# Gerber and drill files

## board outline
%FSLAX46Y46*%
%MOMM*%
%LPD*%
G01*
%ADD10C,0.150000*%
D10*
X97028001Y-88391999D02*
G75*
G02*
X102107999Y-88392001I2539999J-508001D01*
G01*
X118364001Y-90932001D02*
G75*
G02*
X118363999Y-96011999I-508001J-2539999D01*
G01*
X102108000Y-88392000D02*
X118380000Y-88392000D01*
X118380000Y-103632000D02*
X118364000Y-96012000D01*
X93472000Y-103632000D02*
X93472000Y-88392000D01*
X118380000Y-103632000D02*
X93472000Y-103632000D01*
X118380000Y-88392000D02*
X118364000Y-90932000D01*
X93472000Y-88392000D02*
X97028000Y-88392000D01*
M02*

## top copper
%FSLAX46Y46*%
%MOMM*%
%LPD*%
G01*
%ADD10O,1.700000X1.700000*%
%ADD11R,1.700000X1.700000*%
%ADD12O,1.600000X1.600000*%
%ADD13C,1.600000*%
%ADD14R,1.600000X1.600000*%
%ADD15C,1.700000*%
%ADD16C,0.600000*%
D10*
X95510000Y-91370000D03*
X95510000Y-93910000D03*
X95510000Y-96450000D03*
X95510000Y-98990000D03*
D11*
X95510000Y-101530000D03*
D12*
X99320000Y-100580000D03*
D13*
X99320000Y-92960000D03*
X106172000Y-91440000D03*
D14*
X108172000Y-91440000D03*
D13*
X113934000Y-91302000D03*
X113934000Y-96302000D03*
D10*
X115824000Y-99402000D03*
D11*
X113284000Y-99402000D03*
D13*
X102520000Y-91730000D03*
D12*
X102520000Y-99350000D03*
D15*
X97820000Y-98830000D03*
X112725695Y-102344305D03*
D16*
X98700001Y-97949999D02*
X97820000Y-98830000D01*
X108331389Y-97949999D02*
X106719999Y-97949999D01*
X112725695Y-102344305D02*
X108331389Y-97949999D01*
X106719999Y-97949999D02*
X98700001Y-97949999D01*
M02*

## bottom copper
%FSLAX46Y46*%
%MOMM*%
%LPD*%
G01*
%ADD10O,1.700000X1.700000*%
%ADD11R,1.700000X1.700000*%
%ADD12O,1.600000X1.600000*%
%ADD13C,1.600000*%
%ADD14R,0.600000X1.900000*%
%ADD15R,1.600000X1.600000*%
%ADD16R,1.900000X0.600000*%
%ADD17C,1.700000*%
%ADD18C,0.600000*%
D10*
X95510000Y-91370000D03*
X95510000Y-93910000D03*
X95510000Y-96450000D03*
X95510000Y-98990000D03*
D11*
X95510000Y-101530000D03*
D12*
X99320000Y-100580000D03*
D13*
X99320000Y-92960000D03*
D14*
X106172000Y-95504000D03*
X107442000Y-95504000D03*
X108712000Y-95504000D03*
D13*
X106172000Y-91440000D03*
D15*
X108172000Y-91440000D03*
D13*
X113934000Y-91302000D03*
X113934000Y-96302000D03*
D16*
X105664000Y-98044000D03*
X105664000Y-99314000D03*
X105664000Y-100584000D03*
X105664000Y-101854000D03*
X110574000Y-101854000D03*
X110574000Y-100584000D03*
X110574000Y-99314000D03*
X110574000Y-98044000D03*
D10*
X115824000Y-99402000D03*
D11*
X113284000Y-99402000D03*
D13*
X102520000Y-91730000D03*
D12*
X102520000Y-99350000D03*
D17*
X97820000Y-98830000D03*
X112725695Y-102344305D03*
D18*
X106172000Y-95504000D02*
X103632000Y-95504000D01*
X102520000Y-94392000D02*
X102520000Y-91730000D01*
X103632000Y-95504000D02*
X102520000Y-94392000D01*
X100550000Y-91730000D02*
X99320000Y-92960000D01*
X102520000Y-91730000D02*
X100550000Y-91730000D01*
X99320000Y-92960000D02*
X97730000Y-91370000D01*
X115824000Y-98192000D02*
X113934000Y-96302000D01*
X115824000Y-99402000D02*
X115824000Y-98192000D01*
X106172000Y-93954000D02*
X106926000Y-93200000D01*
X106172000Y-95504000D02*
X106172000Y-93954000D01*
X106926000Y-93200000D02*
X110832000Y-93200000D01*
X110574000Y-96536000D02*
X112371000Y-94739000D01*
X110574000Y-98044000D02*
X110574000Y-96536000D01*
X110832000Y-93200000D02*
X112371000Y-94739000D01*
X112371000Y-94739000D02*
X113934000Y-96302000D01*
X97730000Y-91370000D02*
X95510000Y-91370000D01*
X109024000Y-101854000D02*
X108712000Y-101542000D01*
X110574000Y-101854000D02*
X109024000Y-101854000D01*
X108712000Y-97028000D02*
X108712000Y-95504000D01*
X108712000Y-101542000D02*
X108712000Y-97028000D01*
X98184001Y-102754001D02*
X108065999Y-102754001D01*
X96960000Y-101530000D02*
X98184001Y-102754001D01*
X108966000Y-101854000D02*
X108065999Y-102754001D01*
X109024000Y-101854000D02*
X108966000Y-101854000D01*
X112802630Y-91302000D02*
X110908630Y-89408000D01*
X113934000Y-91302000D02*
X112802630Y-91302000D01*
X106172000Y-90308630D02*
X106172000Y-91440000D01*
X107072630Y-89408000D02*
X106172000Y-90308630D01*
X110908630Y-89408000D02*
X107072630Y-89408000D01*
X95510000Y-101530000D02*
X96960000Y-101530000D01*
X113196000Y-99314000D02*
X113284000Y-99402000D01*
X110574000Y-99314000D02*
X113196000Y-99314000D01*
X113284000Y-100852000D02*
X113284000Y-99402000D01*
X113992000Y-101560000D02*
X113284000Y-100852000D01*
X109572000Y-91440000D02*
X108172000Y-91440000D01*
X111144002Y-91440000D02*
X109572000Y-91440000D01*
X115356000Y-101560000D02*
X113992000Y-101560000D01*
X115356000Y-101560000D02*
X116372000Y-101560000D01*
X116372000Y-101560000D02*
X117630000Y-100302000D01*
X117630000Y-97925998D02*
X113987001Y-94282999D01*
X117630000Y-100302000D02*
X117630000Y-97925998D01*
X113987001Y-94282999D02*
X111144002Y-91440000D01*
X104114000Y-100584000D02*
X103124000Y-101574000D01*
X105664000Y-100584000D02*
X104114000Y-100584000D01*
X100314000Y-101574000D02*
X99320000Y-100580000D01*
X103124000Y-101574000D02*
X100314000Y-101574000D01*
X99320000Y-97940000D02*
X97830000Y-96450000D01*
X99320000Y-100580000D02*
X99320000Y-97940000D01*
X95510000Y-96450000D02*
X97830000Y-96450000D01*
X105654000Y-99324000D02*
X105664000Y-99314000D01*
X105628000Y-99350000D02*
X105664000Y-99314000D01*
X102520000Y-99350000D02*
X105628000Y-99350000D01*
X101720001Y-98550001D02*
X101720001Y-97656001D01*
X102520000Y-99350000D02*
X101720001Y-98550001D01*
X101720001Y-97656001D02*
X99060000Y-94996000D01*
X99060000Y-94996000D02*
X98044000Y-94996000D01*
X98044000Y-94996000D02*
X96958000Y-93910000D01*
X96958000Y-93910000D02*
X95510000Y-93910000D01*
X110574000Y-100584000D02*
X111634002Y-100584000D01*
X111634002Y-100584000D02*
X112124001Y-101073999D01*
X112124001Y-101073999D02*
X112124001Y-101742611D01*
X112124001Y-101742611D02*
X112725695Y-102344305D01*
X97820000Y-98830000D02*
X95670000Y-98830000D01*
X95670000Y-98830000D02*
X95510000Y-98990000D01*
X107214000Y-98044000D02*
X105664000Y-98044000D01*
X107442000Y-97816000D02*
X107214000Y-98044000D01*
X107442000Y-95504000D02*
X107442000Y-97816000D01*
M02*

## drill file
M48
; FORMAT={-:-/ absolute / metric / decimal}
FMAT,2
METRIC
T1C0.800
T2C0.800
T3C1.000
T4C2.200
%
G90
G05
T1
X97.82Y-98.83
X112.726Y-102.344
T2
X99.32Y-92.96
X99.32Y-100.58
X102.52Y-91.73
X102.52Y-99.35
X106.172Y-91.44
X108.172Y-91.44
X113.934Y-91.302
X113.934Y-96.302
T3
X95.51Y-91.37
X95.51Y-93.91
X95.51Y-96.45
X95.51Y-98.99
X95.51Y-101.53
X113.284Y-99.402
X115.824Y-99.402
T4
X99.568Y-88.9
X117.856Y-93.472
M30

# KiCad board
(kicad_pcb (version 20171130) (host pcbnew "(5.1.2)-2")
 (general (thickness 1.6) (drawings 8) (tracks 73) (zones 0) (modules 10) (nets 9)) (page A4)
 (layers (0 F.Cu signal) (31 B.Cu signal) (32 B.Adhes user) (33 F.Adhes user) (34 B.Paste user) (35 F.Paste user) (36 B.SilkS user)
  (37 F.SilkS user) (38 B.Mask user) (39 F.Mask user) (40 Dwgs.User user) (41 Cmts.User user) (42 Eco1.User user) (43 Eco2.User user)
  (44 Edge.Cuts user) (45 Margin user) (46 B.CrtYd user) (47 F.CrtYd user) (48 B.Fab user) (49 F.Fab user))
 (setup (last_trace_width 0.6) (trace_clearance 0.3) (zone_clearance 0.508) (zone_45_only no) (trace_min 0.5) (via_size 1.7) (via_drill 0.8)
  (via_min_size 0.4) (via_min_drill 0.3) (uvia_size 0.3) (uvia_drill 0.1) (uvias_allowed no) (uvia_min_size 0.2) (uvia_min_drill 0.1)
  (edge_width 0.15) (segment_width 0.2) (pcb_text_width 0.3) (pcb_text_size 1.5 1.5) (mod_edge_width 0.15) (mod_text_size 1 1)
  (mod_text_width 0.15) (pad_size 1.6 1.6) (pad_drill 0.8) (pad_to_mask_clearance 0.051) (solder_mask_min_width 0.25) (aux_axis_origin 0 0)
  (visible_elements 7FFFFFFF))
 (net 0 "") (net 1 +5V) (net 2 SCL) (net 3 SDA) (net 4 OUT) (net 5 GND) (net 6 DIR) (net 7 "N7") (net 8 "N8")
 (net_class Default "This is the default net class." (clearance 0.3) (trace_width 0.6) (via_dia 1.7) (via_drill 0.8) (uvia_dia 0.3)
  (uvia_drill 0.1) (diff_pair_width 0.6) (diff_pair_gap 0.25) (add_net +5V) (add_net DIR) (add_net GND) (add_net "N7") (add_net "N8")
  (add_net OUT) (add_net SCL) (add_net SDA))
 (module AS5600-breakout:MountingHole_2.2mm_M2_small (layer F.Cu) (at 99.568 88.9)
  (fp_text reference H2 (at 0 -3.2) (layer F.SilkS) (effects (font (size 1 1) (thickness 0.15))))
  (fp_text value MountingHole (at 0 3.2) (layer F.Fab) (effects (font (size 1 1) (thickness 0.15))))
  (pad 1 np_thru_hole circle (at 0 0) (size 2.2 2.2) (drill 2.2) (layers *.Cu *.Mask)))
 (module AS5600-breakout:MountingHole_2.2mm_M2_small (layer F.Cu) (at 117.856 93.472)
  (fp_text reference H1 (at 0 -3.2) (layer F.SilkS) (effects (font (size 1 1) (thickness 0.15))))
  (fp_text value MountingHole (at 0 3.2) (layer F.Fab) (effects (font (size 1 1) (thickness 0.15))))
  (pad 1 np_thru_hole circle (at 0 0) (size 2.2 2.2) (drill 2.2) (layers *.Cu *.Mask)))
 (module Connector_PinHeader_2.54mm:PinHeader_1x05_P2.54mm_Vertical (layer F.Cu) (at 95.51 101.53 180)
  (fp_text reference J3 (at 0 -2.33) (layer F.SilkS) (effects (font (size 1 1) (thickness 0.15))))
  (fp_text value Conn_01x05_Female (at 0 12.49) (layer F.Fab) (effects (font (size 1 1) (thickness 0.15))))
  (pad 5 thru_hole oval (at 0 10.16 180) (size 1.7 1.7) (drill 1) (layers *.Cu *.Mask) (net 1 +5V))
  (pad 4 thru_hole oval (at 0 7.62 180) (size 1.7 1.7) (drill 1) (layers *.Cu *.Mask) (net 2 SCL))
  (pad 3 thru_hole oval (at 0 5.08 180) (size 1.7 1.7) (drill 1) (layers *.Cu *.Mask) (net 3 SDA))
  (pad 2 thru_hole oval (at 0 2.54 180) (size 1.7 1.7) (drill 1) (layers *.Cu *.Mask) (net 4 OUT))
  (pad 1 thru_hole rect (at 0 0 180) (size 1.7 1.7) (drill 1) (layers *.Cu *.Mask) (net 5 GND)))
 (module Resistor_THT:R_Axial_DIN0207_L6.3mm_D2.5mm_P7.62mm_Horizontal (layer F.Cu) (at 99.32 92.96 270)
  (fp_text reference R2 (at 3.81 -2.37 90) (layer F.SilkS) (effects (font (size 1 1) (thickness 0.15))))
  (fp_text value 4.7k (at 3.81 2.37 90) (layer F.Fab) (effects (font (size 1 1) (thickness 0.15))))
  (pad 2 thru_hole oval (at 7.62 0 270) (size 1.6 1.6) (drill 0.8) (layers *.Cu *.Mask) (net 3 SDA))
  (pad 1 thru_hole circle (at 0 0 270) (size 1.6 1.6) (drill 0.8) (layers *.Cu *.Mask) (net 1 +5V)))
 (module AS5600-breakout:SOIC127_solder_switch (layer B.Cu) (at 106.807 93.049 90)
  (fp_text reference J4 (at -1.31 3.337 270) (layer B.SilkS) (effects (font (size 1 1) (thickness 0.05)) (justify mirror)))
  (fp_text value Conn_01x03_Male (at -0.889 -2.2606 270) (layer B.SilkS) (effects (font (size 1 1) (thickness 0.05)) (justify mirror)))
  (pad 3 smd rect (at -2.455 -0.635 90) (size 1.9 0.6) (layers B.Cu B.Paste B.Mask) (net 1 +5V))
  (pad 2 smd rect (at -2.455 0.635 90) (size 1.9 0.6) (layers B.Cu B.Paste B.Mask) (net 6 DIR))
  (pad 1 smd rect (at -2.455 1.905 90) (size 1.9 0.6) (layers B.Cu B.Paste B.Mask) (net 5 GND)))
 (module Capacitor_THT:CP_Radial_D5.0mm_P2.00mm (layer F.Cu) (at 108.172 91.44 180)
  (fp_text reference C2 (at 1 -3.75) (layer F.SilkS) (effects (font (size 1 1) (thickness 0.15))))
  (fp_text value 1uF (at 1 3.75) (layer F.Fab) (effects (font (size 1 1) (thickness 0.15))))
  (pad 2 thru_hole circle (at 2 0 180) (size 1.6 1.6) (drill 0.8) (layers *.Cu *.Mask) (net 5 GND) (clearance 0.2))
  (pad 1 thru_hole rect (at 0 0 180) (size 1.6 1.6) (drill 0.8) (layers *.Cu *.Mask) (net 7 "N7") (clearance 0.2)))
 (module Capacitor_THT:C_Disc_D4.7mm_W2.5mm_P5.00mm (layer F.Cu) (at 113.934 96.302 90)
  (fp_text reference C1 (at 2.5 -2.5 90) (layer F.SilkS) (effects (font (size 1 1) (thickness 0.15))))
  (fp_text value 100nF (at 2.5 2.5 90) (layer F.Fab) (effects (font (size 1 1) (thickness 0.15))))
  (pad 2 thru_hole circle (at 5 0 90) (size 1.6 1.6) (drill 0.8) (layers *.Cu *.Mask) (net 5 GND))
  (pad 1 thru_hole circle (at 0 0 90) (size 1.6 1.6) (drill 0.8) (layers *.Cu *.Mask) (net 1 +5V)))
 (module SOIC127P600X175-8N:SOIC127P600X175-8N (layer B.Cu) (at 108.119 99.949 180)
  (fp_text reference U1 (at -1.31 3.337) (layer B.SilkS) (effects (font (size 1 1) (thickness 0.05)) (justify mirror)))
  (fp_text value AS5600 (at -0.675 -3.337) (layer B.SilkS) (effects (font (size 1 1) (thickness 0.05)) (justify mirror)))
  (pad 8 smd rect (at 2.455 1.905 180) (size 1.9 0.6) (layers B.Cu B.Paste B.Mask) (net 6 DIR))
  (pad 7 smd rect (at 2.455 0.635 180) (size 1.9 0.6) (layers B.Cu B.Paste B.Mask) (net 2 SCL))
  (pad 6 smd rect (at 2.455 -0.635 180) (size 1.9 0.6) (layers B.Cu B.Paste B.Mask) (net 3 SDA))
  (pad 5 smd rect (at 2.455 -1.905 180) (size 1.9 0.6) (layers B.Cu B.Paste B.Mask) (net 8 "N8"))
  (pad 4 smd rect (at -2.455 -1.905 180) (size 1.9 0.6) (layers B.Cu B.Paste B.Mask) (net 5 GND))
  (pad 3 smd rect (at -2.455 -0.635 180) (size 1.9 0.6) (layers B.Cu B.Paste B.Mask) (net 4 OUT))
  (pad 2 smd rect (at -2.455 0.635 180) (size 1.9 0.6) (layers B.Cu B.Paste B.Mask) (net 7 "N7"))
  (pad 1 smd rect (at -2.455 1.905 180) (size 1.9 0.6) (layers B.Cu B.Paste B.Mask) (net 1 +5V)))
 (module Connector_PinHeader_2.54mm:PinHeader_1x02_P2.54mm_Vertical (layer F.Cu) (at 113.284 99.402 90)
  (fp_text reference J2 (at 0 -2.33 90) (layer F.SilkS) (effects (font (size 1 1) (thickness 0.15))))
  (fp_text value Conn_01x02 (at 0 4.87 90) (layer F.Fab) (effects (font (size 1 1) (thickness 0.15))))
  (pad 2 thru_hole oval (at 0 2.54 90) (size 1.7 1.7) (drill 1) (layers *.Cu *.Mask) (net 1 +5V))
  (pad 1 thru_hole rect (at 0 0 90) (size 1.7 1.7) (drill 1) (layers *.Cu *.Mask) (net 7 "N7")))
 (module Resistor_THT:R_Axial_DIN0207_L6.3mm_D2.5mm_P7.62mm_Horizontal (layer F.Cu) (at 102.52 91.73 270)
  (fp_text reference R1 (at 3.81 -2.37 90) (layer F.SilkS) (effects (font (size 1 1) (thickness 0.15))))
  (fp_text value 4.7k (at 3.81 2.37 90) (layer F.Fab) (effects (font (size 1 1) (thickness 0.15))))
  (pad 1 thru_hole circle (at 0 0 270) (size 1.6 1.6) (drill 0.8) (layers *.Cu *.Mask) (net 1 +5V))
  (pad 2 thru_hole oval (at 7.62 0 270) (size 1.6 1.6) (drill 0.8) (layers *.Cu *.Mask) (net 2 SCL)))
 (gr_arc (start 99.568 88.9) (end 102.107999 88.392001) (angle -157.3801351) (layer Edge.Cuts) (width 0.15))
 (gr_arc (start 117.856 93.472) (end 118.363999 96.011999) (angle -157.3801351) (layer Edge.Cuts) (width 0.15))
 (gr_line (start 102.108 88.392) (end 118.38 88.392) (layer Edge.Cuts) (width 0.15))
 (gr_line (start 118.38 103.632) (end 118.364 96.012) (layer Edge.Cuts) (width 0.15))
 (gr_line (start 93.472 103.632) (end 93.472 88.392) (layer Edge.Cuts) (width 0.15))
 (gr_line (start 118.38 103.632) (end 93.472 103.632) (layer Edge.Cuts) (width 0.15))
 (gr_line (start 118.38 88.392) (end 118.364 90.932) (layer Edge.Cuts) (width 0.15))
 (gr_line (start 93.472 88.392) (end 97.028 88.392) (layer Edge.Cuts) (width 0.15))
 (segment (start 106.172 95.504) (end 103.632 95.504) (width 0.6) (layer B.Cu) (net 1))
 (segment (start 102.52 94.392) (end 102.52 91.73) (width 0.6) (layer B.Cu) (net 1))
 (segment (start 103.632 95.504) (end 102.52 94.392) (width 0.6) (layer B.Cu) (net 1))
 (segment (start 100.55 91.73) (end 99.32 92.96) (width 0.6) (layer B.Cu) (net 1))
 (segment (start 102.52 91.73) (end 100.55 91.73) (width 0.6) (layer B.Cu) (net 1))
 (segment (start 99.32 92.96) (end 97.73 91.37) (width 0.6) (layer B.Cu) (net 1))
 (segment (start 115.824 98.192) (end 113.934 96.302) (width 0.6) (layer B.Cu) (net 1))
 (segment (start 115.824 99.402) (end 115.824 98.192) (width 0.6) (layer B.Cu) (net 1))
 (segment (start 106.172 93.954) (end 106.926 93.2) (width 0.6) (layer B.Cu) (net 1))
 (segment (start 106.172 95.504) (end 106.172 93.954) (width 0.6) (layer B.Cu) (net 1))
 (segment (start 106.926 93.2) (end 110.832 93.2) (width 0.6) (layer B.Cu) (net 1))
 (segment (start 110.574 96.536) (end 112.371 94.739) (width 0.6) (layer B.Cu) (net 1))
 (segment (start 110.574 98.044) (end 110.574 96.536) (width 0.6) (layer B.Cu) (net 1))
 (segment (start 110.832 93.2) (end 112.371 94.739) (width 0.6) (layer B.Cu) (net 1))
 (segment (start 112.371 94.739) (end 113.934 96.302) (width 0.6) (layer B.Cu) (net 1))
 (segment (start 97.73 91.37) (end 95.51 91.37) (width 0.6) (layer B.Cu) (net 1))
 (segment (start 109.024 101.854) (end 108.712 101.542) (width 0.6) (layer B.Cu) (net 5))
 (segment (start 110.574 101.854) (end 109.024 101.854) (width 0.6) (layer B.Cu) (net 5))
 (segment (start 108.712 97.028) (end 108.712 95.504) (width 0.6) (layer B.Cu) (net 5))
 (segment (start 108.712 101.542) (end 108.712 97.028) (width 0.6) (layer B.Cu) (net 5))
 (segment (start 98.184001 102.754001) (end 108.065999 102.754001) (width 0.6) (layer B.Cu) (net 5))
 (segment (start 96.96 101.53) (end 98.184001 102.754001) (width 0.6) (layer B.Cu) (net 5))
 (segment (start 108.966 101.854) (end 108.065999 102.754001) (width 0.6) (layer B.Cu) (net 5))
 (segment (start 109.024 101.854) (end 108.966 101.854) (width 0.6) (layer B.Cu) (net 5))
 (segment (start 112.80263 91.302) (end 110.90863 89.408) (width 0.6) (layer B.Cu) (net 5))
 (segment (start 113.934 91.302) (end 112.80263 91.302) (width 0.6) (layer B.Cu) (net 5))
 (segment (start 106.172 90.30863) (end 106.172 91.44) (width 0.6) (layer B.Cu) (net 5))
 (segment (start 107.07263 89.408) (end 106.172 90.30863) (width 0.6) (layer B.Cu) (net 5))
 (segment (start 110.90863 89.408) (end 107.07263 89.408) (width 0.6) (layer B.Cu) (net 5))
 (segment (start 95.51 101.53) (end 96.96 101.53) (width 0.6) (layer B.Cu) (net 5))
 (segment (start 113.196 99.314) (end 113.284 99.402) (width 0.6) (layer B.Cu) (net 7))
 (segment (start 110.574 99.314) (end 113.196 99.314) (width 0.6) (layer B.Cu) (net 7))
 (segment (start 113.284 100.852) (end 113.284 99.402) (width 0.6) (layer B.Cu) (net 7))
 (segment (start 113.992 101.56) (end 113.284 100.852) (width 0.6) (layer B.Cu) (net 7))
 (segment (start 109.572 91.44) (end 108.172 91.44) (width 0.6) (layer B.Cu) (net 7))
 (segment (start 111.144002 91.44) (end 109.572 91.44) (width 0.6) (layer B.Cu) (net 7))
 (segment (start 115.356 101.56) (end 113.992 101.56) (width 0.6) (layer B.Cu) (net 7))
 (segment (start 115.356 101.56) (end 116.372 101.56) (width 0.6) (layer B.Cu) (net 7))
 (segment (start 116.372 101.56) (end 117.63 100.302) (width 0.6) (layer B.Cu) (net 7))
 (segment (start 117.63 97.925998) (end 113.987001 94.282999) (width 0.6) (layer B.Cu) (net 7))
 (segment (start 117.63 100.302) (end 117.63 97.925998) (width 0.6) (layer B.Cu) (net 7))
 (segment (start 113.987001 94.282999) (end 111.144002 91.44) (width 0.6) (layer B.Cu) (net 7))
 (segment (start 104.114 100.584) (end 103.124 101.574) (width 0.6) (layer B.Cu) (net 3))
 (segment (start 105.664 100.584) (end 104.114 100.584) (width 0.6) (layer B.Cu) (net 3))
 (segment (start 100.314 101.574) (end 99.32 100.58) (width 0.6) (layer B.Cu) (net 3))
 (segment (start 103.124 101.574) (end 100.314 101.574) (width 0.6) (layer B.Cu) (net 3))
 (segment (start 99.32 97.94) (end 97.83 96.45) (width 0.6) (layer B.Cu) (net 3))
 (segment (start 99.32 100.58) (end 99.32 97.94) (width 0.6) (layer B.Cu) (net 3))
 (segment (start 95.51 96.45) (end 97.83 96.45) (width 0.6) (layer B.Cu) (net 3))
 (segment (start 105.654 99.324) (end 105.664 99.314) (width 0.6) (layer B.Cu) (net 2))
 (segment (start 105.628 99.35) (end 105.664 99.314) (width 0.6) (layer B.Cu) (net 2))
 (segment (start 102.52 99.35) (end 105.628 99.35) (width 0.6) (layer B.Cu) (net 2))
 (segment (start 101.720001 98.550001) (end 101.720001 97.656001) (width 0.6) (layer B.Cu) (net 2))
 (segment (start 102.52 99.35) (end 101.720001 98.550001) (width 0.6) (layer B.Cu) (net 2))
 (segment (start 101.720001 97.656001) (end 99.06 94.996) (width 0.6) (layer B.Cu) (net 2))
 (segment (start 99.06 94.996) (end 98.044 94.996) (width 0.6) (layer B.Cu) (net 2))
 (segment (start 98.044 94.996) (end 96.958 93.91) (width 0.6) (layer B.Cu) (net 2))
 (segment (start 96.958 93.91) (end 95.51 93.91) (width 0.6) (layer B.Cu) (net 2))
 (segment (start 110.574 100.584) (end 111.634002 100.584) (width 0.6) (layer B.Cu) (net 4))
 (segment (start 111.634002 100.584) (end 112.124001 101.073999) (width 0.6) (layer B.Cu) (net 4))
 (via (at 97.82 98.83) (size 1.7) (drill 0.8) (layers F.Cu B.Cu) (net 4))
 (segment (start 98.700001 97.949999) (end 97.82 98.83) (width 0.6) (layer F.Cu) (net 4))
 (via (at 112.725695 102.344305) (size 1.7) (drill 0.8) (layers F.Cu B.Cu) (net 4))
 (segment (start 112.124001 101.073999) (end 112.124001 101.742611) (width 0.6) (layer B.Cu) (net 4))
 (segment (start 112.124001 101.742611) (end 112.725695 102.344305) (width 0.6) (layer B.Cu) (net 4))
 (segment (start 108.331389 97.949999) (end 106.719999 97.949999) (width 0.6) (layer F.Cu) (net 4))
 (segment (start 112.725695 102.344305) (end 108.331389 97.949999) (width 0.6) (layer F.Cu) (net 4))
 (segment (start 106.719999 97.949999) (end 98.700001 97.949999) (width 0.6) (layer F.Cu) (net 4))
 (segment (start 97.82 98.83) (end 95.67 98.83) (width 0.6) (layer B.Cu) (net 4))
 (segment (start 95.67 98.83) (end 95.51 98.99) (width 0.6) (layer B.Cu) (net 4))
 (segment (start 107.214 98.044) (end 105.664 98.044) (width 0.6) (layer B.Cu) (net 6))
 (segment (start 107.442 97.816) (end 107.214 98.044) (width 0.6) (layer B.Cu) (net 6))
 (segment (start 107.442 95.504) (end 107.442 97.816) (width 0.6) (layer B.Cu) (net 6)))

